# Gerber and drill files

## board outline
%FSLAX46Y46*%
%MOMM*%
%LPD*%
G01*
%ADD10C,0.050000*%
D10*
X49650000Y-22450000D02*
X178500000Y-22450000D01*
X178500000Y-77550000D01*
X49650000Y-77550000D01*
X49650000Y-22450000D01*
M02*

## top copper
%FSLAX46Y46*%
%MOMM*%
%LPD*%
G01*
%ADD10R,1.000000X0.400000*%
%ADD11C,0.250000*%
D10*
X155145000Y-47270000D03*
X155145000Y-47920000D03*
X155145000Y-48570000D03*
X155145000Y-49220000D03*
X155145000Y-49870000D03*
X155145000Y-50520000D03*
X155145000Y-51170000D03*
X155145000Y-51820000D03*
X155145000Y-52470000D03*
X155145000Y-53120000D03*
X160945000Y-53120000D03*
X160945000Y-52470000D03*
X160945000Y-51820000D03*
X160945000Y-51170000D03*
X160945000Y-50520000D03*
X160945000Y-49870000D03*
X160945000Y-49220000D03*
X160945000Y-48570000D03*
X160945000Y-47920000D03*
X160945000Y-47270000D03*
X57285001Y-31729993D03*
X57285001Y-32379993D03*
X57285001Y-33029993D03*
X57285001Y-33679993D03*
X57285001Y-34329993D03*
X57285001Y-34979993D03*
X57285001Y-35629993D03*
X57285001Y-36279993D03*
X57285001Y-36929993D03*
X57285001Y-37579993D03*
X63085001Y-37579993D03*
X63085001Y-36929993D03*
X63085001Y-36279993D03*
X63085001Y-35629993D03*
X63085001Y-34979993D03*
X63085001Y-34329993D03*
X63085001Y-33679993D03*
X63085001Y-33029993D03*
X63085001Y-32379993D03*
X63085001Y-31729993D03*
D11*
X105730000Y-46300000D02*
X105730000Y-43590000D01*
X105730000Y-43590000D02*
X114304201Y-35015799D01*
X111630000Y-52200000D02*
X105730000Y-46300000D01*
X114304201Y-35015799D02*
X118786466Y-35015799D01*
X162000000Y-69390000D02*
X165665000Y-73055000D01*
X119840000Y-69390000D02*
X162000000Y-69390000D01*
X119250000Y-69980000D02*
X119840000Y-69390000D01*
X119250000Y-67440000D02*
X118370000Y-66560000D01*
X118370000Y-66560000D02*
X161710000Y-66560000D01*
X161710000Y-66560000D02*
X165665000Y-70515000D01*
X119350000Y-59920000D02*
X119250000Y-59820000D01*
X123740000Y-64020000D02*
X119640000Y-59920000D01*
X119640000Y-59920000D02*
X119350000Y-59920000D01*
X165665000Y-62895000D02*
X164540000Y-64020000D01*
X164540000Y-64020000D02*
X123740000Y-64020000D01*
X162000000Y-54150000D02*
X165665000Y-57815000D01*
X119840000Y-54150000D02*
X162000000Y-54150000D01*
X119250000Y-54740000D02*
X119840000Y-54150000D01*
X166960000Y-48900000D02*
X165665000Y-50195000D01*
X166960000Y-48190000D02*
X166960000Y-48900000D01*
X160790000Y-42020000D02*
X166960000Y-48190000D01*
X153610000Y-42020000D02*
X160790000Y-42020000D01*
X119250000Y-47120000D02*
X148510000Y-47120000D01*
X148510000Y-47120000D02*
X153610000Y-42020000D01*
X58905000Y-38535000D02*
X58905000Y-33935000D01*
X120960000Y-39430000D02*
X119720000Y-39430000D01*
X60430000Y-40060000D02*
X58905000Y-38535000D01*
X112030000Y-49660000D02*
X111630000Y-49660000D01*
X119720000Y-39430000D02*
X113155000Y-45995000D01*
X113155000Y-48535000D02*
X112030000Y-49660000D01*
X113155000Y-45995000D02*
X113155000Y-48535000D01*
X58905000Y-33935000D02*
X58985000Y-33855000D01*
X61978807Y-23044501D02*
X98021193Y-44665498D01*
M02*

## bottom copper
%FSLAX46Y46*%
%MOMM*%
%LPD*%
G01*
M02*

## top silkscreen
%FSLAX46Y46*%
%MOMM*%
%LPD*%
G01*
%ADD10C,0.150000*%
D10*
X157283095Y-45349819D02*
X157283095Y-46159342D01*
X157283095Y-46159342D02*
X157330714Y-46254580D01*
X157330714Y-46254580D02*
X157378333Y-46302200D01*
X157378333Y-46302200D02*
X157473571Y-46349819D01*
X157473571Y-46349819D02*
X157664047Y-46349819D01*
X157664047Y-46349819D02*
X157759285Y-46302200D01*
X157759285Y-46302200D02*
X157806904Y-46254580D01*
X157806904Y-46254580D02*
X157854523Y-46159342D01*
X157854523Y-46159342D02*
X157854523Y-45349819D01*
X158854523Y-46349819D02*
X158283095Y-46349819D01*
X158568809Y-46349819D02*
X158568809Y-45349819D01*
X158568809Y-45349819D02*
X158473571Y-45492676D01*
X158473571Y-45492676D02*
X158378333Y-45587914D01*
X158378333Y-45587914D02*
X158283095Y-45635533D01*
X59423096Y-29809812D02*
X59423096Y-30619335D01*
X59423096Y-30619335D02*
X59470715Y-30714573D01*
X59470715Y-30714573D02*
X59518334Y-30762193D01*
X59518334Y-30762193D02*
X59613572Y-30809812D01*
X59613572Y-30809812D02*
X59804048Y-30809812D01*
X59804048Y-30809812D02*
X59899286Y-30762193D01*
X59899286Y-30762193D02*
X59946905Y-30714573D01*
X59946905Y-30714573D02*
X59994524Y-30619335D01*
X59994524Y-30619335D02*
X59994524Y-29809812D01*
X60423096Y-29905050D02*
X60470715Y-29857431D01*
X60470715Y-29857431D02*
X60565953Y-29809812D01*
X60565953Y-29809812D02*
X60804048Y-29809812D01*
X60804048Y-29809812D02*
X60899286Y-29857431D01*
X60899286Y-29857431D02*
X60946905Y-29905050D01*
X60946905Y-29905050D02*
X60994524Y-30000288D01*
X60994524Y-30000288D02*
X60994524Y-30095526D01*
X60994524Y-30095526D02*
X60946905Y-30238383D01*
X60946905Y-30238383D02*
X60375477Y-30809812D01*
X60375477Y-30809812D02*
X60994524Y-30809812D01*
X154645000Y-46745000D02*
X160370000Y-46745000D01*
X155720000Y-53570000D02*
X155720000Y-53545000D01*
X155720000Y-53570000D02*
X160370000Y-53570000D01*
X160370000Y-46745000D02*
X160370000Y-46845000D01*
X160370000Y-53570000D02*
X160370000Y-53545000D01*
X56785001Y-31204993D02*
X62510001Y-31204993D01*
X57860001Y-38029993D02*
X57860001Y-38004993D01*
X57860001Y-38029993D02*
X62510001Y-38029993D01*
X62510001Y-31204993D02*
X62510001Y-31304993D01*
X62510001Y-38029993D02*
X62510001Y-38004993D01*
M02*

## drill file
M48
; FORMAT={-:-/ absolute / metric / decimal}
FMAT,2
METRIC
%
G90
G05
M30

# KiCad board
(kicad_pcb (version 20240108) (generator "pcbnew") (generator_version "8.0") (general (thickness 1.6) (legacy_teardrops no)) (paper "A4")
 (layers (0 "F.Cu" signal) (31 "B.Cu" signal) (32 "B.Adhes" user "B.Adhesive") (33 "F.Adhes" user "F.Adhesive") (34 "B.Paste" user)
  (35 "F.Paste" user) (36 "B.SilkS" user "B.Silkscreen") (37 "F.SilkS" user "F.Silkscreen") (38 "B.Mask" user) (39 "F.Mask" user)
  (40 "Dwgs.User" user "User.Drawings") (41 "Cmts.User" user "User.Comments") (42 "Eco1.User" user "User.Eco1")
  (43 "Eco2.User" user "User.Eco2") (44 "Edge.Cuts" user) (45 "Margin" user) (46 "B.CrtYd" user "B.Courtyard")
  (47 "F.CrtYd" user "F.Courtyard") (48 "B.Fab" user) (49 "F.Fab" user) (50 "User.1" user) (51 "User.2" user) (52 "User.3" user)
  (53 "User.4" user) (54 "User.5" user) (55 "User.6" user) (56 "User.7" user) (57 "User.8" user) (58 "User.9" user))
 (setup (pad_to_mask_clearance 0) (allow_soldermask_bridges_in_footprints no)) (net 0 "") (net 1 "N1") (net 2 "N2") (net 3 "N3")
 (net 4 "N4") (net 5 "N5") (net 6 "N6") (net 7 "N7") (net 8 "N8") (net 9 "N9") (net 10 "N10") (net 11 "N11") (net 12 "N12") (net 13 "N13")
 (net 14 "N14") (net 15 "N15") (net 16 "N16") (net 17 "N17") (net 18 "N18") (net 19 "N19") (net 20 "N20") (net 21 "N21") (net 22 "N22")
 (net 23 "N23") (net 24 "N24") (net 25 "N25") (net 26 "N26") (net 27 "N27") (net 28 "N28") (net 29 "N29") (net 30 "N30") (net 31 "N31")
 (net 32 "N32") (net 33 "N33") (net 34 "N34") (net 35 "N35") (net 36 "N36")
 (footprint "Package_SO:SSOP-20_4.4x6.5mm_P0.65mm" (layer "F.Cu") (at 158.045 50.195)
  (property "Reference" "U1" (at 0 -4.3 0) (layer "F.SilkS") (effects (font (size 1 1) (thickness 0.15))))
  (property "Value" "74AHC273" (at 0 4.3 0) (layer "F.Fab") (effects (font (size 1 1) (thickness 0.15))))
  (fp_line (start -3.4 -3.45) (end 2.325 -3.45) (stroke (width 0.15) (type solid)) (layer "F.SilkS"))
  (fp_line (start -2.325 3.375) (end -2.325 3.35) (stroke (width 0.15) (type solid)) (layer "F.SilkS"))
  (fp_line (start -2.325 3.375) (end 2.325 3.375) (stroke (width 0.15) (type solid)) (layer "F.SilkS"))
  (fp_line (start 2.325 -3.45) (end 2.325 -3.35) (stroke (width 0.15) (type solid)) (layer "F.SilkS"))
  (fp_line (start 2.325 3.375) (end 2.325 3.35) (stroke (width 0.15) (type solid)) (layer "F.SilkS"))
  (pad "1" smd rect (at -2.9 -2.925) (size 1 0.4) (layers "F.Cu" "F.Paste" "F.Mask") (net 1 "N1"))
  (pad "2" smd rect (at -2.9 -2.275) (size 1 0.4) (layers "F.Cu" "F.Paste" "F.Mask") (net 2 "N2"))
  (pad "3" smd rect (at -2.9 -1.625) (size 1 0.4) (layers "F.Cu" "F.Paste" "F.Mask") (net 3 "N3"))
  (pad "4" smd rect (at -2.9 -0.975) (size 1 0.4) (layers "F.Cu" "F.Paste" "F.Mask") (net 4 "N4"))
  (pad "5" smd rect (at -2.9 -0.325) (size 1 0.4) (layers "F.Cu" "F.Paste" "F.Mask") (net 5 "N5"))
  (pad "6" smd rect (at -2.9 0.325) (size 1 0.4) (layers "F.Cu" "F.Paste" "F.Mask") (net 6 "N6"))
  (pad "7" smd rect (at -2.9 0.975) (size 1 0.4) (layers "F.Cu" "F.Paste" "F.Mask") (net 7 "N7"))
  (pad "8" smd rect (at -2.9 1.625) (size 1 0.4) (layers "F.Cu" "F.Paste" "F.Mask") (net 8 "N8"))
  (pad "9" smd rect (at -2.9 2.275) (size 1 0.4) (layers "F.Cu" "F.Paste" "F.Mask") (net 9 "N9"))
  (pad "10" smd rect (at -2.9 2.925) (size 1 0.4) (layers "F.Cu" "F.Paste" "F.Mask") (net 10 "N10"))
  (pad "11" smd rect (at 2.9 2.925) (size 1 0.4) (layers "F.Cu" "F.Paste" "F.Mask") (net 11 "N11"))
  (pad "12" smd rect (at 2.9 2.275) (size 1 0.4) (layers "F.Cu" "F.Paste" "F.Mask") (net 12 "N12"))
  (pad "13" smd rect (at 2.9 1.625) (size 1 0.4) (layers "F.Cu" "F.Paste" "F.Mask") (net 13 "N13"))
  (pad "14" smd rect (at 2.9 0.975) (size 1 0.4) (layers "F.Cu" "F.Paste" "F.Mask") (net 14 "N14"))
  (pad "15" smd rect (at 2.9 0.325) (size 1 0.4) (layers "F.Cu" "F.Paste" "F.Mask") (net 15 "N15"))
  (pad "16" smd rect (at 2.9 -0.325) (size 1 0.4) (layers "F.Cu" "F.Paste" "F.Mask") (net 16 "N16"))
  (pad "17" smd rect (at 2.9 -0.975) (size 1 0.4) (layers "F.Cu" "F.Paste" "F.Mask") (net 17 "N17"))
  (pad "18" smd rect (at 2.9 -1.625) (size 1 0.4) (layers "F.Cu" "F.Paste" "F.Mask") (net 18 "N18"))
  (pad "19" smd rect (at 2.9 -2.275) (size 1 0.4) (layers "F.Cu" "F.Paste" "F.Mask") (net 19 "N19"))
  (pad "20" smd rect (at 2.9 -2.925) (size 1 0.4) (layers "F.Cu" "F.Paste" "F.Mask") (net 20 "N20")))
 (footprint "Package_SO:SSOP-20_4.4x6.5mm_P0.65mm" (layer "F.Cu") (at 60.185001 34.654993)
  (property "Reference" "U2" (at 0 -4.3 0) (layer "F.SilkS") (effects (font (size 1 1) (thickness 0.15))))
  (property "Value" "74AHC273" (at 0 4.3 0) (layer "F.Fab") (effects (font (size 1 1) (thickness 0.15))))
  (fp_line (start -3.4 -3.45) (end 2.325 -3.45) (stroke (width 0.15) (type solid)) (layer "F.SilkS"))
  (fp_line (start -2.325 3.375) (end -2.325 3.35) (stroke (width 0.15) (type solid)) (layer "F.SilkS"))
  (fp_line (start -2.325 3.375) (end 2.325 3.375) (stroke (width 0.15) (type solid)) (layer "F.SilkS"))
  (fp_line (start 2.325 -3.45) (end 2.325 -3.35) (stroke (width 0.15) (type solid)) (layer "F.SilkS"))
  (fp_line (start 2.325 3.375) (end 2.325 3.35) (stroke (width 0.15) (type solid)) (layer "F.SilkS"))
  (pad "1" smd rect (at -2.9 -2.925) (size 1 0.4) (layers "F.Cu" "F.Paste" "F.Mask") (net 9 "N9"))
  (pad "2" smd rect (at -2.9 -2.275) (size 1 0.4) (layers "F.Cu" "F.Paste" "F.Mask") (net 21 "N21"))
  (pad "3" smd rect (at -2.9 -1.625) (size 1 0.4) (layers "F.Cu" "F.Paste" "F.Mask") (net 2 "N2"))
  (pad "4" smd rect (at -2.9 -0.975) (size 1 0.4) (layers "F.Cu" "F.Paste" "F.Mask") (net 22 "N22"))
  (pad "5" smd rect (at -2.9 -0.325) (size 1 0.4) (layers "F.Cu" "F.Paste" "F.Mask") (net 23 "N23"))
  (pad "6" smd rect (at -2.9 0.325) (size 1 0.4) (layers "F.Cu" "F.Paste" "F.Mask") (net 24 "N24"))
  (pad "7" smd rect (at -2.9 0.975) (size 1 0.4) (layers "F.Cu" "F.Paste" "F.Mask") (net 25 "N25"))
  (pad "8" smd rect (at -2.9 1.625) (size 1 0.4) (layers "F.Cu" "F.Paste" "F.Mask") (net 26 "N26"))
  (pad "9" smd rect (at -2.9 2.275) (size 1 0.4) (layers "F.Cu" "F.Paste" "F.Mask") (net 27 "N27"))
  (pad "10" smd rect (at -2.9 2.925) (size 1 0.4) (layers "F.Cu" "F.Paste" "F.Mask") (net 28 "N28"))
  (pad "11" smd rect (at 2.9 2.925) (size 1 0.4) (layers "F.Cu" "F.Paste" "F.Mask") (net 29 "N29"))
  (pad "12" smd rect (at 2.9 2.275) (size 1 0.4) (layers "F.Cu" "F.Paste" "F.Mask") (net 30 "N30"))
  (pad "13" smd rect (at 2.9 1.625) (size 1 0.4) (layers "F.Cu" "F.Paste" "F.Mask") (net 6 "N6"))
  (pad "14" smd rect (at 2.9 0.975) (size 1 0.4) (layers "F.Cu" "F.Paste" "F.Mask") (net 9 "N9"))
  (pad "15" smd rect (at 2.9 0.325) (size 1 0.4) (layers "F.Cu" "F.Paste" "F.Mask") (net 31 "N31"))
  (pad "16" smd rect (at 2.9 -0.325) (size 1 0.4) (layers "F.Cu" "F.Paste" "F.Mask") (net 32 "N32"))
  (pad "17" smd rect (at 2.9 -0.975) (size 1 0.4) (layers "F.Cu" "F.Paste" "F.Mask") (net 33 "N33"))
  (pad "18" smd rect (at 2.9 -1.625) (size 1 0.4) (layers "F.Cu" "F.Paste" "F.Mask") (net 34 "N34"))
  (pad "19" smd rect (at 2.9 -2.275) (size 1 0.4) (layers "F.Cu" "F.Paste" "F.Mask") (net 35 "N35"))
  (pad "20" smd rect (at 2.9 -2.925) (size 1 0.4) (layers "F.Cu" "F.Paste" "F.Mask") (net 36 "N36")))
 (gr_rect (start 49.65 22.45) (end 178.5 77.55) (stroke (width 0.05) (type default)) (fill none) (layer "Edge.Cuts"))
 (segment (start 105.73 46.3) (end 105.73 43.59) (width 0.25) (layer "F.Cu") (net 3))
 (segment (start 105.73 43.59) (end 114.304201 35.015799) (width 0.25) (layer "F.Cu") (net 3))
 (segment (start 111.63 52.2) (end 105.73 46.3) (width 0.25) (layer "F.Cu") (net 3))
 (segment (start 114.304201 35.015799) (end 118.786466 35.015799) (width 0.25) (layer "F.Cu") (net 3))
 (segment (start 162 69.39) (end 165.665 73.055) (width 0.25) (layer "F.Cu") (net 11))
 (segment (start 119.84 69.39) (end 162 69.39) (width 0.25) (layer "F.Cu") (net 11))
 (segment (start 119.25 69.98) (end 119.84 69.39) (width 0.25) (layer "F.Cu") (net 11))
 (segment (start 119.25 67.44) (end 118.37 66.56) (width 0.25) (layer "F.Cu") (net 12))
 (segment (start 118.37 66.56) (end 161.71 66.56) (width 0.25) (layer "F.Cu") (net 12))
 (segment (start 161.71 66.56) (end 165.665 70.515) (width 0.25) (layer "F.Cu") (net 12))
 (segment (start 119.35 59.92) (end 119.25 59.82) (width 0.25) (layer "F.Cu") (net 15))
 (segment (start 123.74 64.02) (end 119.64 59.92) (width 0.25) (layer "F.Cu") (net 15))
 (segment (start 119.64 59.92) (end 119.35 59.92) (width 0.25) (layer "F.Cu") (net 15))
 (segment (start 165.665 62.895) (end 164.54 64.02) (width 0.25) (layer "F.Cu") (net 15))
 (segment (start 164.54 64.02) (end 123.74 64.02) (width 0.25) (layer "F.Cu") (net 15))
 (segment (start 162 54.15) (end 165.665 57.815) (width 0.25) (layer "F.Cu") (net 17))
 (segment (start 119.84 54.15) (end 162 54.15) (width 0.25) (layer "F.Cu") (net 17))
 (segment (start 119.25 54.74) (end 119.84 54.15) (width 0.25) (layer "F.Cu") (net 17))
 (segment (start 166.96 48.9) (end 165.665 50.195) (width 0.25) (layer "F.Cu") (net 20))
 (segment (start 166.96 48.19) (end 166.96 48.9) (width 0.25) (layer "F.Cu") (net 20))
 (segment (start 160.79 42.02) (end 166.96 48.19) (width 0.25) (layer "F.Cu") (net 20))
 (segment (start 153.61 42.02) (end 160.79 42.02) (width 0.25) (layer "F.Cu") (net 20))
 (segment (start 119.25 47.12) (end 148.51 47.12) (width 0.25) (layer "F.Cu") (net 20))
 (segment (start 148.51 47.12) (end 153.61 42.02) (width 0.25) (layer "F.Cu") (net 20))
 (segment (start 58.905 38.535) (end 58.905 33.935) (width 0.25) (layer "F.Cu") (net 2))
 (segment (start 120.96 39.43) (end 119.72 39.43) (width 0.25) (layer "F.Cu") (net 2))
 (segment (start 60.43 40.06) (end 58.905 38.535) (width 0.25) (layer "F.Cu") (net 2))
 (segment (start 112.03 49.66) (end 111.63 49.66) (width 0.25) (layer "F.Cu") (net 2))
 (segment (start 119.72 39.43) (end 113.155 45.995) (width 0.25) (layer "F.Cu") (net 2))
 (segment (start 113.155 48.535) (end 112.03 49.66) (width 0.25) (layer "F.Cu") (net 2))
 (segment (start 113.155 45.995) (end 113.155 48.535) (width 0.25) (layer "F.Cu") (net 2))
 (segment (start 58.905 33.935) (end 58.985 33.855) (width 0.25) (layer "F.Cu") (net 2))
 (segment (start 61.978807 23.044501) (end 98.021193 44.665498) (width 0.25) (layer "F.Cu") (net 2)))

